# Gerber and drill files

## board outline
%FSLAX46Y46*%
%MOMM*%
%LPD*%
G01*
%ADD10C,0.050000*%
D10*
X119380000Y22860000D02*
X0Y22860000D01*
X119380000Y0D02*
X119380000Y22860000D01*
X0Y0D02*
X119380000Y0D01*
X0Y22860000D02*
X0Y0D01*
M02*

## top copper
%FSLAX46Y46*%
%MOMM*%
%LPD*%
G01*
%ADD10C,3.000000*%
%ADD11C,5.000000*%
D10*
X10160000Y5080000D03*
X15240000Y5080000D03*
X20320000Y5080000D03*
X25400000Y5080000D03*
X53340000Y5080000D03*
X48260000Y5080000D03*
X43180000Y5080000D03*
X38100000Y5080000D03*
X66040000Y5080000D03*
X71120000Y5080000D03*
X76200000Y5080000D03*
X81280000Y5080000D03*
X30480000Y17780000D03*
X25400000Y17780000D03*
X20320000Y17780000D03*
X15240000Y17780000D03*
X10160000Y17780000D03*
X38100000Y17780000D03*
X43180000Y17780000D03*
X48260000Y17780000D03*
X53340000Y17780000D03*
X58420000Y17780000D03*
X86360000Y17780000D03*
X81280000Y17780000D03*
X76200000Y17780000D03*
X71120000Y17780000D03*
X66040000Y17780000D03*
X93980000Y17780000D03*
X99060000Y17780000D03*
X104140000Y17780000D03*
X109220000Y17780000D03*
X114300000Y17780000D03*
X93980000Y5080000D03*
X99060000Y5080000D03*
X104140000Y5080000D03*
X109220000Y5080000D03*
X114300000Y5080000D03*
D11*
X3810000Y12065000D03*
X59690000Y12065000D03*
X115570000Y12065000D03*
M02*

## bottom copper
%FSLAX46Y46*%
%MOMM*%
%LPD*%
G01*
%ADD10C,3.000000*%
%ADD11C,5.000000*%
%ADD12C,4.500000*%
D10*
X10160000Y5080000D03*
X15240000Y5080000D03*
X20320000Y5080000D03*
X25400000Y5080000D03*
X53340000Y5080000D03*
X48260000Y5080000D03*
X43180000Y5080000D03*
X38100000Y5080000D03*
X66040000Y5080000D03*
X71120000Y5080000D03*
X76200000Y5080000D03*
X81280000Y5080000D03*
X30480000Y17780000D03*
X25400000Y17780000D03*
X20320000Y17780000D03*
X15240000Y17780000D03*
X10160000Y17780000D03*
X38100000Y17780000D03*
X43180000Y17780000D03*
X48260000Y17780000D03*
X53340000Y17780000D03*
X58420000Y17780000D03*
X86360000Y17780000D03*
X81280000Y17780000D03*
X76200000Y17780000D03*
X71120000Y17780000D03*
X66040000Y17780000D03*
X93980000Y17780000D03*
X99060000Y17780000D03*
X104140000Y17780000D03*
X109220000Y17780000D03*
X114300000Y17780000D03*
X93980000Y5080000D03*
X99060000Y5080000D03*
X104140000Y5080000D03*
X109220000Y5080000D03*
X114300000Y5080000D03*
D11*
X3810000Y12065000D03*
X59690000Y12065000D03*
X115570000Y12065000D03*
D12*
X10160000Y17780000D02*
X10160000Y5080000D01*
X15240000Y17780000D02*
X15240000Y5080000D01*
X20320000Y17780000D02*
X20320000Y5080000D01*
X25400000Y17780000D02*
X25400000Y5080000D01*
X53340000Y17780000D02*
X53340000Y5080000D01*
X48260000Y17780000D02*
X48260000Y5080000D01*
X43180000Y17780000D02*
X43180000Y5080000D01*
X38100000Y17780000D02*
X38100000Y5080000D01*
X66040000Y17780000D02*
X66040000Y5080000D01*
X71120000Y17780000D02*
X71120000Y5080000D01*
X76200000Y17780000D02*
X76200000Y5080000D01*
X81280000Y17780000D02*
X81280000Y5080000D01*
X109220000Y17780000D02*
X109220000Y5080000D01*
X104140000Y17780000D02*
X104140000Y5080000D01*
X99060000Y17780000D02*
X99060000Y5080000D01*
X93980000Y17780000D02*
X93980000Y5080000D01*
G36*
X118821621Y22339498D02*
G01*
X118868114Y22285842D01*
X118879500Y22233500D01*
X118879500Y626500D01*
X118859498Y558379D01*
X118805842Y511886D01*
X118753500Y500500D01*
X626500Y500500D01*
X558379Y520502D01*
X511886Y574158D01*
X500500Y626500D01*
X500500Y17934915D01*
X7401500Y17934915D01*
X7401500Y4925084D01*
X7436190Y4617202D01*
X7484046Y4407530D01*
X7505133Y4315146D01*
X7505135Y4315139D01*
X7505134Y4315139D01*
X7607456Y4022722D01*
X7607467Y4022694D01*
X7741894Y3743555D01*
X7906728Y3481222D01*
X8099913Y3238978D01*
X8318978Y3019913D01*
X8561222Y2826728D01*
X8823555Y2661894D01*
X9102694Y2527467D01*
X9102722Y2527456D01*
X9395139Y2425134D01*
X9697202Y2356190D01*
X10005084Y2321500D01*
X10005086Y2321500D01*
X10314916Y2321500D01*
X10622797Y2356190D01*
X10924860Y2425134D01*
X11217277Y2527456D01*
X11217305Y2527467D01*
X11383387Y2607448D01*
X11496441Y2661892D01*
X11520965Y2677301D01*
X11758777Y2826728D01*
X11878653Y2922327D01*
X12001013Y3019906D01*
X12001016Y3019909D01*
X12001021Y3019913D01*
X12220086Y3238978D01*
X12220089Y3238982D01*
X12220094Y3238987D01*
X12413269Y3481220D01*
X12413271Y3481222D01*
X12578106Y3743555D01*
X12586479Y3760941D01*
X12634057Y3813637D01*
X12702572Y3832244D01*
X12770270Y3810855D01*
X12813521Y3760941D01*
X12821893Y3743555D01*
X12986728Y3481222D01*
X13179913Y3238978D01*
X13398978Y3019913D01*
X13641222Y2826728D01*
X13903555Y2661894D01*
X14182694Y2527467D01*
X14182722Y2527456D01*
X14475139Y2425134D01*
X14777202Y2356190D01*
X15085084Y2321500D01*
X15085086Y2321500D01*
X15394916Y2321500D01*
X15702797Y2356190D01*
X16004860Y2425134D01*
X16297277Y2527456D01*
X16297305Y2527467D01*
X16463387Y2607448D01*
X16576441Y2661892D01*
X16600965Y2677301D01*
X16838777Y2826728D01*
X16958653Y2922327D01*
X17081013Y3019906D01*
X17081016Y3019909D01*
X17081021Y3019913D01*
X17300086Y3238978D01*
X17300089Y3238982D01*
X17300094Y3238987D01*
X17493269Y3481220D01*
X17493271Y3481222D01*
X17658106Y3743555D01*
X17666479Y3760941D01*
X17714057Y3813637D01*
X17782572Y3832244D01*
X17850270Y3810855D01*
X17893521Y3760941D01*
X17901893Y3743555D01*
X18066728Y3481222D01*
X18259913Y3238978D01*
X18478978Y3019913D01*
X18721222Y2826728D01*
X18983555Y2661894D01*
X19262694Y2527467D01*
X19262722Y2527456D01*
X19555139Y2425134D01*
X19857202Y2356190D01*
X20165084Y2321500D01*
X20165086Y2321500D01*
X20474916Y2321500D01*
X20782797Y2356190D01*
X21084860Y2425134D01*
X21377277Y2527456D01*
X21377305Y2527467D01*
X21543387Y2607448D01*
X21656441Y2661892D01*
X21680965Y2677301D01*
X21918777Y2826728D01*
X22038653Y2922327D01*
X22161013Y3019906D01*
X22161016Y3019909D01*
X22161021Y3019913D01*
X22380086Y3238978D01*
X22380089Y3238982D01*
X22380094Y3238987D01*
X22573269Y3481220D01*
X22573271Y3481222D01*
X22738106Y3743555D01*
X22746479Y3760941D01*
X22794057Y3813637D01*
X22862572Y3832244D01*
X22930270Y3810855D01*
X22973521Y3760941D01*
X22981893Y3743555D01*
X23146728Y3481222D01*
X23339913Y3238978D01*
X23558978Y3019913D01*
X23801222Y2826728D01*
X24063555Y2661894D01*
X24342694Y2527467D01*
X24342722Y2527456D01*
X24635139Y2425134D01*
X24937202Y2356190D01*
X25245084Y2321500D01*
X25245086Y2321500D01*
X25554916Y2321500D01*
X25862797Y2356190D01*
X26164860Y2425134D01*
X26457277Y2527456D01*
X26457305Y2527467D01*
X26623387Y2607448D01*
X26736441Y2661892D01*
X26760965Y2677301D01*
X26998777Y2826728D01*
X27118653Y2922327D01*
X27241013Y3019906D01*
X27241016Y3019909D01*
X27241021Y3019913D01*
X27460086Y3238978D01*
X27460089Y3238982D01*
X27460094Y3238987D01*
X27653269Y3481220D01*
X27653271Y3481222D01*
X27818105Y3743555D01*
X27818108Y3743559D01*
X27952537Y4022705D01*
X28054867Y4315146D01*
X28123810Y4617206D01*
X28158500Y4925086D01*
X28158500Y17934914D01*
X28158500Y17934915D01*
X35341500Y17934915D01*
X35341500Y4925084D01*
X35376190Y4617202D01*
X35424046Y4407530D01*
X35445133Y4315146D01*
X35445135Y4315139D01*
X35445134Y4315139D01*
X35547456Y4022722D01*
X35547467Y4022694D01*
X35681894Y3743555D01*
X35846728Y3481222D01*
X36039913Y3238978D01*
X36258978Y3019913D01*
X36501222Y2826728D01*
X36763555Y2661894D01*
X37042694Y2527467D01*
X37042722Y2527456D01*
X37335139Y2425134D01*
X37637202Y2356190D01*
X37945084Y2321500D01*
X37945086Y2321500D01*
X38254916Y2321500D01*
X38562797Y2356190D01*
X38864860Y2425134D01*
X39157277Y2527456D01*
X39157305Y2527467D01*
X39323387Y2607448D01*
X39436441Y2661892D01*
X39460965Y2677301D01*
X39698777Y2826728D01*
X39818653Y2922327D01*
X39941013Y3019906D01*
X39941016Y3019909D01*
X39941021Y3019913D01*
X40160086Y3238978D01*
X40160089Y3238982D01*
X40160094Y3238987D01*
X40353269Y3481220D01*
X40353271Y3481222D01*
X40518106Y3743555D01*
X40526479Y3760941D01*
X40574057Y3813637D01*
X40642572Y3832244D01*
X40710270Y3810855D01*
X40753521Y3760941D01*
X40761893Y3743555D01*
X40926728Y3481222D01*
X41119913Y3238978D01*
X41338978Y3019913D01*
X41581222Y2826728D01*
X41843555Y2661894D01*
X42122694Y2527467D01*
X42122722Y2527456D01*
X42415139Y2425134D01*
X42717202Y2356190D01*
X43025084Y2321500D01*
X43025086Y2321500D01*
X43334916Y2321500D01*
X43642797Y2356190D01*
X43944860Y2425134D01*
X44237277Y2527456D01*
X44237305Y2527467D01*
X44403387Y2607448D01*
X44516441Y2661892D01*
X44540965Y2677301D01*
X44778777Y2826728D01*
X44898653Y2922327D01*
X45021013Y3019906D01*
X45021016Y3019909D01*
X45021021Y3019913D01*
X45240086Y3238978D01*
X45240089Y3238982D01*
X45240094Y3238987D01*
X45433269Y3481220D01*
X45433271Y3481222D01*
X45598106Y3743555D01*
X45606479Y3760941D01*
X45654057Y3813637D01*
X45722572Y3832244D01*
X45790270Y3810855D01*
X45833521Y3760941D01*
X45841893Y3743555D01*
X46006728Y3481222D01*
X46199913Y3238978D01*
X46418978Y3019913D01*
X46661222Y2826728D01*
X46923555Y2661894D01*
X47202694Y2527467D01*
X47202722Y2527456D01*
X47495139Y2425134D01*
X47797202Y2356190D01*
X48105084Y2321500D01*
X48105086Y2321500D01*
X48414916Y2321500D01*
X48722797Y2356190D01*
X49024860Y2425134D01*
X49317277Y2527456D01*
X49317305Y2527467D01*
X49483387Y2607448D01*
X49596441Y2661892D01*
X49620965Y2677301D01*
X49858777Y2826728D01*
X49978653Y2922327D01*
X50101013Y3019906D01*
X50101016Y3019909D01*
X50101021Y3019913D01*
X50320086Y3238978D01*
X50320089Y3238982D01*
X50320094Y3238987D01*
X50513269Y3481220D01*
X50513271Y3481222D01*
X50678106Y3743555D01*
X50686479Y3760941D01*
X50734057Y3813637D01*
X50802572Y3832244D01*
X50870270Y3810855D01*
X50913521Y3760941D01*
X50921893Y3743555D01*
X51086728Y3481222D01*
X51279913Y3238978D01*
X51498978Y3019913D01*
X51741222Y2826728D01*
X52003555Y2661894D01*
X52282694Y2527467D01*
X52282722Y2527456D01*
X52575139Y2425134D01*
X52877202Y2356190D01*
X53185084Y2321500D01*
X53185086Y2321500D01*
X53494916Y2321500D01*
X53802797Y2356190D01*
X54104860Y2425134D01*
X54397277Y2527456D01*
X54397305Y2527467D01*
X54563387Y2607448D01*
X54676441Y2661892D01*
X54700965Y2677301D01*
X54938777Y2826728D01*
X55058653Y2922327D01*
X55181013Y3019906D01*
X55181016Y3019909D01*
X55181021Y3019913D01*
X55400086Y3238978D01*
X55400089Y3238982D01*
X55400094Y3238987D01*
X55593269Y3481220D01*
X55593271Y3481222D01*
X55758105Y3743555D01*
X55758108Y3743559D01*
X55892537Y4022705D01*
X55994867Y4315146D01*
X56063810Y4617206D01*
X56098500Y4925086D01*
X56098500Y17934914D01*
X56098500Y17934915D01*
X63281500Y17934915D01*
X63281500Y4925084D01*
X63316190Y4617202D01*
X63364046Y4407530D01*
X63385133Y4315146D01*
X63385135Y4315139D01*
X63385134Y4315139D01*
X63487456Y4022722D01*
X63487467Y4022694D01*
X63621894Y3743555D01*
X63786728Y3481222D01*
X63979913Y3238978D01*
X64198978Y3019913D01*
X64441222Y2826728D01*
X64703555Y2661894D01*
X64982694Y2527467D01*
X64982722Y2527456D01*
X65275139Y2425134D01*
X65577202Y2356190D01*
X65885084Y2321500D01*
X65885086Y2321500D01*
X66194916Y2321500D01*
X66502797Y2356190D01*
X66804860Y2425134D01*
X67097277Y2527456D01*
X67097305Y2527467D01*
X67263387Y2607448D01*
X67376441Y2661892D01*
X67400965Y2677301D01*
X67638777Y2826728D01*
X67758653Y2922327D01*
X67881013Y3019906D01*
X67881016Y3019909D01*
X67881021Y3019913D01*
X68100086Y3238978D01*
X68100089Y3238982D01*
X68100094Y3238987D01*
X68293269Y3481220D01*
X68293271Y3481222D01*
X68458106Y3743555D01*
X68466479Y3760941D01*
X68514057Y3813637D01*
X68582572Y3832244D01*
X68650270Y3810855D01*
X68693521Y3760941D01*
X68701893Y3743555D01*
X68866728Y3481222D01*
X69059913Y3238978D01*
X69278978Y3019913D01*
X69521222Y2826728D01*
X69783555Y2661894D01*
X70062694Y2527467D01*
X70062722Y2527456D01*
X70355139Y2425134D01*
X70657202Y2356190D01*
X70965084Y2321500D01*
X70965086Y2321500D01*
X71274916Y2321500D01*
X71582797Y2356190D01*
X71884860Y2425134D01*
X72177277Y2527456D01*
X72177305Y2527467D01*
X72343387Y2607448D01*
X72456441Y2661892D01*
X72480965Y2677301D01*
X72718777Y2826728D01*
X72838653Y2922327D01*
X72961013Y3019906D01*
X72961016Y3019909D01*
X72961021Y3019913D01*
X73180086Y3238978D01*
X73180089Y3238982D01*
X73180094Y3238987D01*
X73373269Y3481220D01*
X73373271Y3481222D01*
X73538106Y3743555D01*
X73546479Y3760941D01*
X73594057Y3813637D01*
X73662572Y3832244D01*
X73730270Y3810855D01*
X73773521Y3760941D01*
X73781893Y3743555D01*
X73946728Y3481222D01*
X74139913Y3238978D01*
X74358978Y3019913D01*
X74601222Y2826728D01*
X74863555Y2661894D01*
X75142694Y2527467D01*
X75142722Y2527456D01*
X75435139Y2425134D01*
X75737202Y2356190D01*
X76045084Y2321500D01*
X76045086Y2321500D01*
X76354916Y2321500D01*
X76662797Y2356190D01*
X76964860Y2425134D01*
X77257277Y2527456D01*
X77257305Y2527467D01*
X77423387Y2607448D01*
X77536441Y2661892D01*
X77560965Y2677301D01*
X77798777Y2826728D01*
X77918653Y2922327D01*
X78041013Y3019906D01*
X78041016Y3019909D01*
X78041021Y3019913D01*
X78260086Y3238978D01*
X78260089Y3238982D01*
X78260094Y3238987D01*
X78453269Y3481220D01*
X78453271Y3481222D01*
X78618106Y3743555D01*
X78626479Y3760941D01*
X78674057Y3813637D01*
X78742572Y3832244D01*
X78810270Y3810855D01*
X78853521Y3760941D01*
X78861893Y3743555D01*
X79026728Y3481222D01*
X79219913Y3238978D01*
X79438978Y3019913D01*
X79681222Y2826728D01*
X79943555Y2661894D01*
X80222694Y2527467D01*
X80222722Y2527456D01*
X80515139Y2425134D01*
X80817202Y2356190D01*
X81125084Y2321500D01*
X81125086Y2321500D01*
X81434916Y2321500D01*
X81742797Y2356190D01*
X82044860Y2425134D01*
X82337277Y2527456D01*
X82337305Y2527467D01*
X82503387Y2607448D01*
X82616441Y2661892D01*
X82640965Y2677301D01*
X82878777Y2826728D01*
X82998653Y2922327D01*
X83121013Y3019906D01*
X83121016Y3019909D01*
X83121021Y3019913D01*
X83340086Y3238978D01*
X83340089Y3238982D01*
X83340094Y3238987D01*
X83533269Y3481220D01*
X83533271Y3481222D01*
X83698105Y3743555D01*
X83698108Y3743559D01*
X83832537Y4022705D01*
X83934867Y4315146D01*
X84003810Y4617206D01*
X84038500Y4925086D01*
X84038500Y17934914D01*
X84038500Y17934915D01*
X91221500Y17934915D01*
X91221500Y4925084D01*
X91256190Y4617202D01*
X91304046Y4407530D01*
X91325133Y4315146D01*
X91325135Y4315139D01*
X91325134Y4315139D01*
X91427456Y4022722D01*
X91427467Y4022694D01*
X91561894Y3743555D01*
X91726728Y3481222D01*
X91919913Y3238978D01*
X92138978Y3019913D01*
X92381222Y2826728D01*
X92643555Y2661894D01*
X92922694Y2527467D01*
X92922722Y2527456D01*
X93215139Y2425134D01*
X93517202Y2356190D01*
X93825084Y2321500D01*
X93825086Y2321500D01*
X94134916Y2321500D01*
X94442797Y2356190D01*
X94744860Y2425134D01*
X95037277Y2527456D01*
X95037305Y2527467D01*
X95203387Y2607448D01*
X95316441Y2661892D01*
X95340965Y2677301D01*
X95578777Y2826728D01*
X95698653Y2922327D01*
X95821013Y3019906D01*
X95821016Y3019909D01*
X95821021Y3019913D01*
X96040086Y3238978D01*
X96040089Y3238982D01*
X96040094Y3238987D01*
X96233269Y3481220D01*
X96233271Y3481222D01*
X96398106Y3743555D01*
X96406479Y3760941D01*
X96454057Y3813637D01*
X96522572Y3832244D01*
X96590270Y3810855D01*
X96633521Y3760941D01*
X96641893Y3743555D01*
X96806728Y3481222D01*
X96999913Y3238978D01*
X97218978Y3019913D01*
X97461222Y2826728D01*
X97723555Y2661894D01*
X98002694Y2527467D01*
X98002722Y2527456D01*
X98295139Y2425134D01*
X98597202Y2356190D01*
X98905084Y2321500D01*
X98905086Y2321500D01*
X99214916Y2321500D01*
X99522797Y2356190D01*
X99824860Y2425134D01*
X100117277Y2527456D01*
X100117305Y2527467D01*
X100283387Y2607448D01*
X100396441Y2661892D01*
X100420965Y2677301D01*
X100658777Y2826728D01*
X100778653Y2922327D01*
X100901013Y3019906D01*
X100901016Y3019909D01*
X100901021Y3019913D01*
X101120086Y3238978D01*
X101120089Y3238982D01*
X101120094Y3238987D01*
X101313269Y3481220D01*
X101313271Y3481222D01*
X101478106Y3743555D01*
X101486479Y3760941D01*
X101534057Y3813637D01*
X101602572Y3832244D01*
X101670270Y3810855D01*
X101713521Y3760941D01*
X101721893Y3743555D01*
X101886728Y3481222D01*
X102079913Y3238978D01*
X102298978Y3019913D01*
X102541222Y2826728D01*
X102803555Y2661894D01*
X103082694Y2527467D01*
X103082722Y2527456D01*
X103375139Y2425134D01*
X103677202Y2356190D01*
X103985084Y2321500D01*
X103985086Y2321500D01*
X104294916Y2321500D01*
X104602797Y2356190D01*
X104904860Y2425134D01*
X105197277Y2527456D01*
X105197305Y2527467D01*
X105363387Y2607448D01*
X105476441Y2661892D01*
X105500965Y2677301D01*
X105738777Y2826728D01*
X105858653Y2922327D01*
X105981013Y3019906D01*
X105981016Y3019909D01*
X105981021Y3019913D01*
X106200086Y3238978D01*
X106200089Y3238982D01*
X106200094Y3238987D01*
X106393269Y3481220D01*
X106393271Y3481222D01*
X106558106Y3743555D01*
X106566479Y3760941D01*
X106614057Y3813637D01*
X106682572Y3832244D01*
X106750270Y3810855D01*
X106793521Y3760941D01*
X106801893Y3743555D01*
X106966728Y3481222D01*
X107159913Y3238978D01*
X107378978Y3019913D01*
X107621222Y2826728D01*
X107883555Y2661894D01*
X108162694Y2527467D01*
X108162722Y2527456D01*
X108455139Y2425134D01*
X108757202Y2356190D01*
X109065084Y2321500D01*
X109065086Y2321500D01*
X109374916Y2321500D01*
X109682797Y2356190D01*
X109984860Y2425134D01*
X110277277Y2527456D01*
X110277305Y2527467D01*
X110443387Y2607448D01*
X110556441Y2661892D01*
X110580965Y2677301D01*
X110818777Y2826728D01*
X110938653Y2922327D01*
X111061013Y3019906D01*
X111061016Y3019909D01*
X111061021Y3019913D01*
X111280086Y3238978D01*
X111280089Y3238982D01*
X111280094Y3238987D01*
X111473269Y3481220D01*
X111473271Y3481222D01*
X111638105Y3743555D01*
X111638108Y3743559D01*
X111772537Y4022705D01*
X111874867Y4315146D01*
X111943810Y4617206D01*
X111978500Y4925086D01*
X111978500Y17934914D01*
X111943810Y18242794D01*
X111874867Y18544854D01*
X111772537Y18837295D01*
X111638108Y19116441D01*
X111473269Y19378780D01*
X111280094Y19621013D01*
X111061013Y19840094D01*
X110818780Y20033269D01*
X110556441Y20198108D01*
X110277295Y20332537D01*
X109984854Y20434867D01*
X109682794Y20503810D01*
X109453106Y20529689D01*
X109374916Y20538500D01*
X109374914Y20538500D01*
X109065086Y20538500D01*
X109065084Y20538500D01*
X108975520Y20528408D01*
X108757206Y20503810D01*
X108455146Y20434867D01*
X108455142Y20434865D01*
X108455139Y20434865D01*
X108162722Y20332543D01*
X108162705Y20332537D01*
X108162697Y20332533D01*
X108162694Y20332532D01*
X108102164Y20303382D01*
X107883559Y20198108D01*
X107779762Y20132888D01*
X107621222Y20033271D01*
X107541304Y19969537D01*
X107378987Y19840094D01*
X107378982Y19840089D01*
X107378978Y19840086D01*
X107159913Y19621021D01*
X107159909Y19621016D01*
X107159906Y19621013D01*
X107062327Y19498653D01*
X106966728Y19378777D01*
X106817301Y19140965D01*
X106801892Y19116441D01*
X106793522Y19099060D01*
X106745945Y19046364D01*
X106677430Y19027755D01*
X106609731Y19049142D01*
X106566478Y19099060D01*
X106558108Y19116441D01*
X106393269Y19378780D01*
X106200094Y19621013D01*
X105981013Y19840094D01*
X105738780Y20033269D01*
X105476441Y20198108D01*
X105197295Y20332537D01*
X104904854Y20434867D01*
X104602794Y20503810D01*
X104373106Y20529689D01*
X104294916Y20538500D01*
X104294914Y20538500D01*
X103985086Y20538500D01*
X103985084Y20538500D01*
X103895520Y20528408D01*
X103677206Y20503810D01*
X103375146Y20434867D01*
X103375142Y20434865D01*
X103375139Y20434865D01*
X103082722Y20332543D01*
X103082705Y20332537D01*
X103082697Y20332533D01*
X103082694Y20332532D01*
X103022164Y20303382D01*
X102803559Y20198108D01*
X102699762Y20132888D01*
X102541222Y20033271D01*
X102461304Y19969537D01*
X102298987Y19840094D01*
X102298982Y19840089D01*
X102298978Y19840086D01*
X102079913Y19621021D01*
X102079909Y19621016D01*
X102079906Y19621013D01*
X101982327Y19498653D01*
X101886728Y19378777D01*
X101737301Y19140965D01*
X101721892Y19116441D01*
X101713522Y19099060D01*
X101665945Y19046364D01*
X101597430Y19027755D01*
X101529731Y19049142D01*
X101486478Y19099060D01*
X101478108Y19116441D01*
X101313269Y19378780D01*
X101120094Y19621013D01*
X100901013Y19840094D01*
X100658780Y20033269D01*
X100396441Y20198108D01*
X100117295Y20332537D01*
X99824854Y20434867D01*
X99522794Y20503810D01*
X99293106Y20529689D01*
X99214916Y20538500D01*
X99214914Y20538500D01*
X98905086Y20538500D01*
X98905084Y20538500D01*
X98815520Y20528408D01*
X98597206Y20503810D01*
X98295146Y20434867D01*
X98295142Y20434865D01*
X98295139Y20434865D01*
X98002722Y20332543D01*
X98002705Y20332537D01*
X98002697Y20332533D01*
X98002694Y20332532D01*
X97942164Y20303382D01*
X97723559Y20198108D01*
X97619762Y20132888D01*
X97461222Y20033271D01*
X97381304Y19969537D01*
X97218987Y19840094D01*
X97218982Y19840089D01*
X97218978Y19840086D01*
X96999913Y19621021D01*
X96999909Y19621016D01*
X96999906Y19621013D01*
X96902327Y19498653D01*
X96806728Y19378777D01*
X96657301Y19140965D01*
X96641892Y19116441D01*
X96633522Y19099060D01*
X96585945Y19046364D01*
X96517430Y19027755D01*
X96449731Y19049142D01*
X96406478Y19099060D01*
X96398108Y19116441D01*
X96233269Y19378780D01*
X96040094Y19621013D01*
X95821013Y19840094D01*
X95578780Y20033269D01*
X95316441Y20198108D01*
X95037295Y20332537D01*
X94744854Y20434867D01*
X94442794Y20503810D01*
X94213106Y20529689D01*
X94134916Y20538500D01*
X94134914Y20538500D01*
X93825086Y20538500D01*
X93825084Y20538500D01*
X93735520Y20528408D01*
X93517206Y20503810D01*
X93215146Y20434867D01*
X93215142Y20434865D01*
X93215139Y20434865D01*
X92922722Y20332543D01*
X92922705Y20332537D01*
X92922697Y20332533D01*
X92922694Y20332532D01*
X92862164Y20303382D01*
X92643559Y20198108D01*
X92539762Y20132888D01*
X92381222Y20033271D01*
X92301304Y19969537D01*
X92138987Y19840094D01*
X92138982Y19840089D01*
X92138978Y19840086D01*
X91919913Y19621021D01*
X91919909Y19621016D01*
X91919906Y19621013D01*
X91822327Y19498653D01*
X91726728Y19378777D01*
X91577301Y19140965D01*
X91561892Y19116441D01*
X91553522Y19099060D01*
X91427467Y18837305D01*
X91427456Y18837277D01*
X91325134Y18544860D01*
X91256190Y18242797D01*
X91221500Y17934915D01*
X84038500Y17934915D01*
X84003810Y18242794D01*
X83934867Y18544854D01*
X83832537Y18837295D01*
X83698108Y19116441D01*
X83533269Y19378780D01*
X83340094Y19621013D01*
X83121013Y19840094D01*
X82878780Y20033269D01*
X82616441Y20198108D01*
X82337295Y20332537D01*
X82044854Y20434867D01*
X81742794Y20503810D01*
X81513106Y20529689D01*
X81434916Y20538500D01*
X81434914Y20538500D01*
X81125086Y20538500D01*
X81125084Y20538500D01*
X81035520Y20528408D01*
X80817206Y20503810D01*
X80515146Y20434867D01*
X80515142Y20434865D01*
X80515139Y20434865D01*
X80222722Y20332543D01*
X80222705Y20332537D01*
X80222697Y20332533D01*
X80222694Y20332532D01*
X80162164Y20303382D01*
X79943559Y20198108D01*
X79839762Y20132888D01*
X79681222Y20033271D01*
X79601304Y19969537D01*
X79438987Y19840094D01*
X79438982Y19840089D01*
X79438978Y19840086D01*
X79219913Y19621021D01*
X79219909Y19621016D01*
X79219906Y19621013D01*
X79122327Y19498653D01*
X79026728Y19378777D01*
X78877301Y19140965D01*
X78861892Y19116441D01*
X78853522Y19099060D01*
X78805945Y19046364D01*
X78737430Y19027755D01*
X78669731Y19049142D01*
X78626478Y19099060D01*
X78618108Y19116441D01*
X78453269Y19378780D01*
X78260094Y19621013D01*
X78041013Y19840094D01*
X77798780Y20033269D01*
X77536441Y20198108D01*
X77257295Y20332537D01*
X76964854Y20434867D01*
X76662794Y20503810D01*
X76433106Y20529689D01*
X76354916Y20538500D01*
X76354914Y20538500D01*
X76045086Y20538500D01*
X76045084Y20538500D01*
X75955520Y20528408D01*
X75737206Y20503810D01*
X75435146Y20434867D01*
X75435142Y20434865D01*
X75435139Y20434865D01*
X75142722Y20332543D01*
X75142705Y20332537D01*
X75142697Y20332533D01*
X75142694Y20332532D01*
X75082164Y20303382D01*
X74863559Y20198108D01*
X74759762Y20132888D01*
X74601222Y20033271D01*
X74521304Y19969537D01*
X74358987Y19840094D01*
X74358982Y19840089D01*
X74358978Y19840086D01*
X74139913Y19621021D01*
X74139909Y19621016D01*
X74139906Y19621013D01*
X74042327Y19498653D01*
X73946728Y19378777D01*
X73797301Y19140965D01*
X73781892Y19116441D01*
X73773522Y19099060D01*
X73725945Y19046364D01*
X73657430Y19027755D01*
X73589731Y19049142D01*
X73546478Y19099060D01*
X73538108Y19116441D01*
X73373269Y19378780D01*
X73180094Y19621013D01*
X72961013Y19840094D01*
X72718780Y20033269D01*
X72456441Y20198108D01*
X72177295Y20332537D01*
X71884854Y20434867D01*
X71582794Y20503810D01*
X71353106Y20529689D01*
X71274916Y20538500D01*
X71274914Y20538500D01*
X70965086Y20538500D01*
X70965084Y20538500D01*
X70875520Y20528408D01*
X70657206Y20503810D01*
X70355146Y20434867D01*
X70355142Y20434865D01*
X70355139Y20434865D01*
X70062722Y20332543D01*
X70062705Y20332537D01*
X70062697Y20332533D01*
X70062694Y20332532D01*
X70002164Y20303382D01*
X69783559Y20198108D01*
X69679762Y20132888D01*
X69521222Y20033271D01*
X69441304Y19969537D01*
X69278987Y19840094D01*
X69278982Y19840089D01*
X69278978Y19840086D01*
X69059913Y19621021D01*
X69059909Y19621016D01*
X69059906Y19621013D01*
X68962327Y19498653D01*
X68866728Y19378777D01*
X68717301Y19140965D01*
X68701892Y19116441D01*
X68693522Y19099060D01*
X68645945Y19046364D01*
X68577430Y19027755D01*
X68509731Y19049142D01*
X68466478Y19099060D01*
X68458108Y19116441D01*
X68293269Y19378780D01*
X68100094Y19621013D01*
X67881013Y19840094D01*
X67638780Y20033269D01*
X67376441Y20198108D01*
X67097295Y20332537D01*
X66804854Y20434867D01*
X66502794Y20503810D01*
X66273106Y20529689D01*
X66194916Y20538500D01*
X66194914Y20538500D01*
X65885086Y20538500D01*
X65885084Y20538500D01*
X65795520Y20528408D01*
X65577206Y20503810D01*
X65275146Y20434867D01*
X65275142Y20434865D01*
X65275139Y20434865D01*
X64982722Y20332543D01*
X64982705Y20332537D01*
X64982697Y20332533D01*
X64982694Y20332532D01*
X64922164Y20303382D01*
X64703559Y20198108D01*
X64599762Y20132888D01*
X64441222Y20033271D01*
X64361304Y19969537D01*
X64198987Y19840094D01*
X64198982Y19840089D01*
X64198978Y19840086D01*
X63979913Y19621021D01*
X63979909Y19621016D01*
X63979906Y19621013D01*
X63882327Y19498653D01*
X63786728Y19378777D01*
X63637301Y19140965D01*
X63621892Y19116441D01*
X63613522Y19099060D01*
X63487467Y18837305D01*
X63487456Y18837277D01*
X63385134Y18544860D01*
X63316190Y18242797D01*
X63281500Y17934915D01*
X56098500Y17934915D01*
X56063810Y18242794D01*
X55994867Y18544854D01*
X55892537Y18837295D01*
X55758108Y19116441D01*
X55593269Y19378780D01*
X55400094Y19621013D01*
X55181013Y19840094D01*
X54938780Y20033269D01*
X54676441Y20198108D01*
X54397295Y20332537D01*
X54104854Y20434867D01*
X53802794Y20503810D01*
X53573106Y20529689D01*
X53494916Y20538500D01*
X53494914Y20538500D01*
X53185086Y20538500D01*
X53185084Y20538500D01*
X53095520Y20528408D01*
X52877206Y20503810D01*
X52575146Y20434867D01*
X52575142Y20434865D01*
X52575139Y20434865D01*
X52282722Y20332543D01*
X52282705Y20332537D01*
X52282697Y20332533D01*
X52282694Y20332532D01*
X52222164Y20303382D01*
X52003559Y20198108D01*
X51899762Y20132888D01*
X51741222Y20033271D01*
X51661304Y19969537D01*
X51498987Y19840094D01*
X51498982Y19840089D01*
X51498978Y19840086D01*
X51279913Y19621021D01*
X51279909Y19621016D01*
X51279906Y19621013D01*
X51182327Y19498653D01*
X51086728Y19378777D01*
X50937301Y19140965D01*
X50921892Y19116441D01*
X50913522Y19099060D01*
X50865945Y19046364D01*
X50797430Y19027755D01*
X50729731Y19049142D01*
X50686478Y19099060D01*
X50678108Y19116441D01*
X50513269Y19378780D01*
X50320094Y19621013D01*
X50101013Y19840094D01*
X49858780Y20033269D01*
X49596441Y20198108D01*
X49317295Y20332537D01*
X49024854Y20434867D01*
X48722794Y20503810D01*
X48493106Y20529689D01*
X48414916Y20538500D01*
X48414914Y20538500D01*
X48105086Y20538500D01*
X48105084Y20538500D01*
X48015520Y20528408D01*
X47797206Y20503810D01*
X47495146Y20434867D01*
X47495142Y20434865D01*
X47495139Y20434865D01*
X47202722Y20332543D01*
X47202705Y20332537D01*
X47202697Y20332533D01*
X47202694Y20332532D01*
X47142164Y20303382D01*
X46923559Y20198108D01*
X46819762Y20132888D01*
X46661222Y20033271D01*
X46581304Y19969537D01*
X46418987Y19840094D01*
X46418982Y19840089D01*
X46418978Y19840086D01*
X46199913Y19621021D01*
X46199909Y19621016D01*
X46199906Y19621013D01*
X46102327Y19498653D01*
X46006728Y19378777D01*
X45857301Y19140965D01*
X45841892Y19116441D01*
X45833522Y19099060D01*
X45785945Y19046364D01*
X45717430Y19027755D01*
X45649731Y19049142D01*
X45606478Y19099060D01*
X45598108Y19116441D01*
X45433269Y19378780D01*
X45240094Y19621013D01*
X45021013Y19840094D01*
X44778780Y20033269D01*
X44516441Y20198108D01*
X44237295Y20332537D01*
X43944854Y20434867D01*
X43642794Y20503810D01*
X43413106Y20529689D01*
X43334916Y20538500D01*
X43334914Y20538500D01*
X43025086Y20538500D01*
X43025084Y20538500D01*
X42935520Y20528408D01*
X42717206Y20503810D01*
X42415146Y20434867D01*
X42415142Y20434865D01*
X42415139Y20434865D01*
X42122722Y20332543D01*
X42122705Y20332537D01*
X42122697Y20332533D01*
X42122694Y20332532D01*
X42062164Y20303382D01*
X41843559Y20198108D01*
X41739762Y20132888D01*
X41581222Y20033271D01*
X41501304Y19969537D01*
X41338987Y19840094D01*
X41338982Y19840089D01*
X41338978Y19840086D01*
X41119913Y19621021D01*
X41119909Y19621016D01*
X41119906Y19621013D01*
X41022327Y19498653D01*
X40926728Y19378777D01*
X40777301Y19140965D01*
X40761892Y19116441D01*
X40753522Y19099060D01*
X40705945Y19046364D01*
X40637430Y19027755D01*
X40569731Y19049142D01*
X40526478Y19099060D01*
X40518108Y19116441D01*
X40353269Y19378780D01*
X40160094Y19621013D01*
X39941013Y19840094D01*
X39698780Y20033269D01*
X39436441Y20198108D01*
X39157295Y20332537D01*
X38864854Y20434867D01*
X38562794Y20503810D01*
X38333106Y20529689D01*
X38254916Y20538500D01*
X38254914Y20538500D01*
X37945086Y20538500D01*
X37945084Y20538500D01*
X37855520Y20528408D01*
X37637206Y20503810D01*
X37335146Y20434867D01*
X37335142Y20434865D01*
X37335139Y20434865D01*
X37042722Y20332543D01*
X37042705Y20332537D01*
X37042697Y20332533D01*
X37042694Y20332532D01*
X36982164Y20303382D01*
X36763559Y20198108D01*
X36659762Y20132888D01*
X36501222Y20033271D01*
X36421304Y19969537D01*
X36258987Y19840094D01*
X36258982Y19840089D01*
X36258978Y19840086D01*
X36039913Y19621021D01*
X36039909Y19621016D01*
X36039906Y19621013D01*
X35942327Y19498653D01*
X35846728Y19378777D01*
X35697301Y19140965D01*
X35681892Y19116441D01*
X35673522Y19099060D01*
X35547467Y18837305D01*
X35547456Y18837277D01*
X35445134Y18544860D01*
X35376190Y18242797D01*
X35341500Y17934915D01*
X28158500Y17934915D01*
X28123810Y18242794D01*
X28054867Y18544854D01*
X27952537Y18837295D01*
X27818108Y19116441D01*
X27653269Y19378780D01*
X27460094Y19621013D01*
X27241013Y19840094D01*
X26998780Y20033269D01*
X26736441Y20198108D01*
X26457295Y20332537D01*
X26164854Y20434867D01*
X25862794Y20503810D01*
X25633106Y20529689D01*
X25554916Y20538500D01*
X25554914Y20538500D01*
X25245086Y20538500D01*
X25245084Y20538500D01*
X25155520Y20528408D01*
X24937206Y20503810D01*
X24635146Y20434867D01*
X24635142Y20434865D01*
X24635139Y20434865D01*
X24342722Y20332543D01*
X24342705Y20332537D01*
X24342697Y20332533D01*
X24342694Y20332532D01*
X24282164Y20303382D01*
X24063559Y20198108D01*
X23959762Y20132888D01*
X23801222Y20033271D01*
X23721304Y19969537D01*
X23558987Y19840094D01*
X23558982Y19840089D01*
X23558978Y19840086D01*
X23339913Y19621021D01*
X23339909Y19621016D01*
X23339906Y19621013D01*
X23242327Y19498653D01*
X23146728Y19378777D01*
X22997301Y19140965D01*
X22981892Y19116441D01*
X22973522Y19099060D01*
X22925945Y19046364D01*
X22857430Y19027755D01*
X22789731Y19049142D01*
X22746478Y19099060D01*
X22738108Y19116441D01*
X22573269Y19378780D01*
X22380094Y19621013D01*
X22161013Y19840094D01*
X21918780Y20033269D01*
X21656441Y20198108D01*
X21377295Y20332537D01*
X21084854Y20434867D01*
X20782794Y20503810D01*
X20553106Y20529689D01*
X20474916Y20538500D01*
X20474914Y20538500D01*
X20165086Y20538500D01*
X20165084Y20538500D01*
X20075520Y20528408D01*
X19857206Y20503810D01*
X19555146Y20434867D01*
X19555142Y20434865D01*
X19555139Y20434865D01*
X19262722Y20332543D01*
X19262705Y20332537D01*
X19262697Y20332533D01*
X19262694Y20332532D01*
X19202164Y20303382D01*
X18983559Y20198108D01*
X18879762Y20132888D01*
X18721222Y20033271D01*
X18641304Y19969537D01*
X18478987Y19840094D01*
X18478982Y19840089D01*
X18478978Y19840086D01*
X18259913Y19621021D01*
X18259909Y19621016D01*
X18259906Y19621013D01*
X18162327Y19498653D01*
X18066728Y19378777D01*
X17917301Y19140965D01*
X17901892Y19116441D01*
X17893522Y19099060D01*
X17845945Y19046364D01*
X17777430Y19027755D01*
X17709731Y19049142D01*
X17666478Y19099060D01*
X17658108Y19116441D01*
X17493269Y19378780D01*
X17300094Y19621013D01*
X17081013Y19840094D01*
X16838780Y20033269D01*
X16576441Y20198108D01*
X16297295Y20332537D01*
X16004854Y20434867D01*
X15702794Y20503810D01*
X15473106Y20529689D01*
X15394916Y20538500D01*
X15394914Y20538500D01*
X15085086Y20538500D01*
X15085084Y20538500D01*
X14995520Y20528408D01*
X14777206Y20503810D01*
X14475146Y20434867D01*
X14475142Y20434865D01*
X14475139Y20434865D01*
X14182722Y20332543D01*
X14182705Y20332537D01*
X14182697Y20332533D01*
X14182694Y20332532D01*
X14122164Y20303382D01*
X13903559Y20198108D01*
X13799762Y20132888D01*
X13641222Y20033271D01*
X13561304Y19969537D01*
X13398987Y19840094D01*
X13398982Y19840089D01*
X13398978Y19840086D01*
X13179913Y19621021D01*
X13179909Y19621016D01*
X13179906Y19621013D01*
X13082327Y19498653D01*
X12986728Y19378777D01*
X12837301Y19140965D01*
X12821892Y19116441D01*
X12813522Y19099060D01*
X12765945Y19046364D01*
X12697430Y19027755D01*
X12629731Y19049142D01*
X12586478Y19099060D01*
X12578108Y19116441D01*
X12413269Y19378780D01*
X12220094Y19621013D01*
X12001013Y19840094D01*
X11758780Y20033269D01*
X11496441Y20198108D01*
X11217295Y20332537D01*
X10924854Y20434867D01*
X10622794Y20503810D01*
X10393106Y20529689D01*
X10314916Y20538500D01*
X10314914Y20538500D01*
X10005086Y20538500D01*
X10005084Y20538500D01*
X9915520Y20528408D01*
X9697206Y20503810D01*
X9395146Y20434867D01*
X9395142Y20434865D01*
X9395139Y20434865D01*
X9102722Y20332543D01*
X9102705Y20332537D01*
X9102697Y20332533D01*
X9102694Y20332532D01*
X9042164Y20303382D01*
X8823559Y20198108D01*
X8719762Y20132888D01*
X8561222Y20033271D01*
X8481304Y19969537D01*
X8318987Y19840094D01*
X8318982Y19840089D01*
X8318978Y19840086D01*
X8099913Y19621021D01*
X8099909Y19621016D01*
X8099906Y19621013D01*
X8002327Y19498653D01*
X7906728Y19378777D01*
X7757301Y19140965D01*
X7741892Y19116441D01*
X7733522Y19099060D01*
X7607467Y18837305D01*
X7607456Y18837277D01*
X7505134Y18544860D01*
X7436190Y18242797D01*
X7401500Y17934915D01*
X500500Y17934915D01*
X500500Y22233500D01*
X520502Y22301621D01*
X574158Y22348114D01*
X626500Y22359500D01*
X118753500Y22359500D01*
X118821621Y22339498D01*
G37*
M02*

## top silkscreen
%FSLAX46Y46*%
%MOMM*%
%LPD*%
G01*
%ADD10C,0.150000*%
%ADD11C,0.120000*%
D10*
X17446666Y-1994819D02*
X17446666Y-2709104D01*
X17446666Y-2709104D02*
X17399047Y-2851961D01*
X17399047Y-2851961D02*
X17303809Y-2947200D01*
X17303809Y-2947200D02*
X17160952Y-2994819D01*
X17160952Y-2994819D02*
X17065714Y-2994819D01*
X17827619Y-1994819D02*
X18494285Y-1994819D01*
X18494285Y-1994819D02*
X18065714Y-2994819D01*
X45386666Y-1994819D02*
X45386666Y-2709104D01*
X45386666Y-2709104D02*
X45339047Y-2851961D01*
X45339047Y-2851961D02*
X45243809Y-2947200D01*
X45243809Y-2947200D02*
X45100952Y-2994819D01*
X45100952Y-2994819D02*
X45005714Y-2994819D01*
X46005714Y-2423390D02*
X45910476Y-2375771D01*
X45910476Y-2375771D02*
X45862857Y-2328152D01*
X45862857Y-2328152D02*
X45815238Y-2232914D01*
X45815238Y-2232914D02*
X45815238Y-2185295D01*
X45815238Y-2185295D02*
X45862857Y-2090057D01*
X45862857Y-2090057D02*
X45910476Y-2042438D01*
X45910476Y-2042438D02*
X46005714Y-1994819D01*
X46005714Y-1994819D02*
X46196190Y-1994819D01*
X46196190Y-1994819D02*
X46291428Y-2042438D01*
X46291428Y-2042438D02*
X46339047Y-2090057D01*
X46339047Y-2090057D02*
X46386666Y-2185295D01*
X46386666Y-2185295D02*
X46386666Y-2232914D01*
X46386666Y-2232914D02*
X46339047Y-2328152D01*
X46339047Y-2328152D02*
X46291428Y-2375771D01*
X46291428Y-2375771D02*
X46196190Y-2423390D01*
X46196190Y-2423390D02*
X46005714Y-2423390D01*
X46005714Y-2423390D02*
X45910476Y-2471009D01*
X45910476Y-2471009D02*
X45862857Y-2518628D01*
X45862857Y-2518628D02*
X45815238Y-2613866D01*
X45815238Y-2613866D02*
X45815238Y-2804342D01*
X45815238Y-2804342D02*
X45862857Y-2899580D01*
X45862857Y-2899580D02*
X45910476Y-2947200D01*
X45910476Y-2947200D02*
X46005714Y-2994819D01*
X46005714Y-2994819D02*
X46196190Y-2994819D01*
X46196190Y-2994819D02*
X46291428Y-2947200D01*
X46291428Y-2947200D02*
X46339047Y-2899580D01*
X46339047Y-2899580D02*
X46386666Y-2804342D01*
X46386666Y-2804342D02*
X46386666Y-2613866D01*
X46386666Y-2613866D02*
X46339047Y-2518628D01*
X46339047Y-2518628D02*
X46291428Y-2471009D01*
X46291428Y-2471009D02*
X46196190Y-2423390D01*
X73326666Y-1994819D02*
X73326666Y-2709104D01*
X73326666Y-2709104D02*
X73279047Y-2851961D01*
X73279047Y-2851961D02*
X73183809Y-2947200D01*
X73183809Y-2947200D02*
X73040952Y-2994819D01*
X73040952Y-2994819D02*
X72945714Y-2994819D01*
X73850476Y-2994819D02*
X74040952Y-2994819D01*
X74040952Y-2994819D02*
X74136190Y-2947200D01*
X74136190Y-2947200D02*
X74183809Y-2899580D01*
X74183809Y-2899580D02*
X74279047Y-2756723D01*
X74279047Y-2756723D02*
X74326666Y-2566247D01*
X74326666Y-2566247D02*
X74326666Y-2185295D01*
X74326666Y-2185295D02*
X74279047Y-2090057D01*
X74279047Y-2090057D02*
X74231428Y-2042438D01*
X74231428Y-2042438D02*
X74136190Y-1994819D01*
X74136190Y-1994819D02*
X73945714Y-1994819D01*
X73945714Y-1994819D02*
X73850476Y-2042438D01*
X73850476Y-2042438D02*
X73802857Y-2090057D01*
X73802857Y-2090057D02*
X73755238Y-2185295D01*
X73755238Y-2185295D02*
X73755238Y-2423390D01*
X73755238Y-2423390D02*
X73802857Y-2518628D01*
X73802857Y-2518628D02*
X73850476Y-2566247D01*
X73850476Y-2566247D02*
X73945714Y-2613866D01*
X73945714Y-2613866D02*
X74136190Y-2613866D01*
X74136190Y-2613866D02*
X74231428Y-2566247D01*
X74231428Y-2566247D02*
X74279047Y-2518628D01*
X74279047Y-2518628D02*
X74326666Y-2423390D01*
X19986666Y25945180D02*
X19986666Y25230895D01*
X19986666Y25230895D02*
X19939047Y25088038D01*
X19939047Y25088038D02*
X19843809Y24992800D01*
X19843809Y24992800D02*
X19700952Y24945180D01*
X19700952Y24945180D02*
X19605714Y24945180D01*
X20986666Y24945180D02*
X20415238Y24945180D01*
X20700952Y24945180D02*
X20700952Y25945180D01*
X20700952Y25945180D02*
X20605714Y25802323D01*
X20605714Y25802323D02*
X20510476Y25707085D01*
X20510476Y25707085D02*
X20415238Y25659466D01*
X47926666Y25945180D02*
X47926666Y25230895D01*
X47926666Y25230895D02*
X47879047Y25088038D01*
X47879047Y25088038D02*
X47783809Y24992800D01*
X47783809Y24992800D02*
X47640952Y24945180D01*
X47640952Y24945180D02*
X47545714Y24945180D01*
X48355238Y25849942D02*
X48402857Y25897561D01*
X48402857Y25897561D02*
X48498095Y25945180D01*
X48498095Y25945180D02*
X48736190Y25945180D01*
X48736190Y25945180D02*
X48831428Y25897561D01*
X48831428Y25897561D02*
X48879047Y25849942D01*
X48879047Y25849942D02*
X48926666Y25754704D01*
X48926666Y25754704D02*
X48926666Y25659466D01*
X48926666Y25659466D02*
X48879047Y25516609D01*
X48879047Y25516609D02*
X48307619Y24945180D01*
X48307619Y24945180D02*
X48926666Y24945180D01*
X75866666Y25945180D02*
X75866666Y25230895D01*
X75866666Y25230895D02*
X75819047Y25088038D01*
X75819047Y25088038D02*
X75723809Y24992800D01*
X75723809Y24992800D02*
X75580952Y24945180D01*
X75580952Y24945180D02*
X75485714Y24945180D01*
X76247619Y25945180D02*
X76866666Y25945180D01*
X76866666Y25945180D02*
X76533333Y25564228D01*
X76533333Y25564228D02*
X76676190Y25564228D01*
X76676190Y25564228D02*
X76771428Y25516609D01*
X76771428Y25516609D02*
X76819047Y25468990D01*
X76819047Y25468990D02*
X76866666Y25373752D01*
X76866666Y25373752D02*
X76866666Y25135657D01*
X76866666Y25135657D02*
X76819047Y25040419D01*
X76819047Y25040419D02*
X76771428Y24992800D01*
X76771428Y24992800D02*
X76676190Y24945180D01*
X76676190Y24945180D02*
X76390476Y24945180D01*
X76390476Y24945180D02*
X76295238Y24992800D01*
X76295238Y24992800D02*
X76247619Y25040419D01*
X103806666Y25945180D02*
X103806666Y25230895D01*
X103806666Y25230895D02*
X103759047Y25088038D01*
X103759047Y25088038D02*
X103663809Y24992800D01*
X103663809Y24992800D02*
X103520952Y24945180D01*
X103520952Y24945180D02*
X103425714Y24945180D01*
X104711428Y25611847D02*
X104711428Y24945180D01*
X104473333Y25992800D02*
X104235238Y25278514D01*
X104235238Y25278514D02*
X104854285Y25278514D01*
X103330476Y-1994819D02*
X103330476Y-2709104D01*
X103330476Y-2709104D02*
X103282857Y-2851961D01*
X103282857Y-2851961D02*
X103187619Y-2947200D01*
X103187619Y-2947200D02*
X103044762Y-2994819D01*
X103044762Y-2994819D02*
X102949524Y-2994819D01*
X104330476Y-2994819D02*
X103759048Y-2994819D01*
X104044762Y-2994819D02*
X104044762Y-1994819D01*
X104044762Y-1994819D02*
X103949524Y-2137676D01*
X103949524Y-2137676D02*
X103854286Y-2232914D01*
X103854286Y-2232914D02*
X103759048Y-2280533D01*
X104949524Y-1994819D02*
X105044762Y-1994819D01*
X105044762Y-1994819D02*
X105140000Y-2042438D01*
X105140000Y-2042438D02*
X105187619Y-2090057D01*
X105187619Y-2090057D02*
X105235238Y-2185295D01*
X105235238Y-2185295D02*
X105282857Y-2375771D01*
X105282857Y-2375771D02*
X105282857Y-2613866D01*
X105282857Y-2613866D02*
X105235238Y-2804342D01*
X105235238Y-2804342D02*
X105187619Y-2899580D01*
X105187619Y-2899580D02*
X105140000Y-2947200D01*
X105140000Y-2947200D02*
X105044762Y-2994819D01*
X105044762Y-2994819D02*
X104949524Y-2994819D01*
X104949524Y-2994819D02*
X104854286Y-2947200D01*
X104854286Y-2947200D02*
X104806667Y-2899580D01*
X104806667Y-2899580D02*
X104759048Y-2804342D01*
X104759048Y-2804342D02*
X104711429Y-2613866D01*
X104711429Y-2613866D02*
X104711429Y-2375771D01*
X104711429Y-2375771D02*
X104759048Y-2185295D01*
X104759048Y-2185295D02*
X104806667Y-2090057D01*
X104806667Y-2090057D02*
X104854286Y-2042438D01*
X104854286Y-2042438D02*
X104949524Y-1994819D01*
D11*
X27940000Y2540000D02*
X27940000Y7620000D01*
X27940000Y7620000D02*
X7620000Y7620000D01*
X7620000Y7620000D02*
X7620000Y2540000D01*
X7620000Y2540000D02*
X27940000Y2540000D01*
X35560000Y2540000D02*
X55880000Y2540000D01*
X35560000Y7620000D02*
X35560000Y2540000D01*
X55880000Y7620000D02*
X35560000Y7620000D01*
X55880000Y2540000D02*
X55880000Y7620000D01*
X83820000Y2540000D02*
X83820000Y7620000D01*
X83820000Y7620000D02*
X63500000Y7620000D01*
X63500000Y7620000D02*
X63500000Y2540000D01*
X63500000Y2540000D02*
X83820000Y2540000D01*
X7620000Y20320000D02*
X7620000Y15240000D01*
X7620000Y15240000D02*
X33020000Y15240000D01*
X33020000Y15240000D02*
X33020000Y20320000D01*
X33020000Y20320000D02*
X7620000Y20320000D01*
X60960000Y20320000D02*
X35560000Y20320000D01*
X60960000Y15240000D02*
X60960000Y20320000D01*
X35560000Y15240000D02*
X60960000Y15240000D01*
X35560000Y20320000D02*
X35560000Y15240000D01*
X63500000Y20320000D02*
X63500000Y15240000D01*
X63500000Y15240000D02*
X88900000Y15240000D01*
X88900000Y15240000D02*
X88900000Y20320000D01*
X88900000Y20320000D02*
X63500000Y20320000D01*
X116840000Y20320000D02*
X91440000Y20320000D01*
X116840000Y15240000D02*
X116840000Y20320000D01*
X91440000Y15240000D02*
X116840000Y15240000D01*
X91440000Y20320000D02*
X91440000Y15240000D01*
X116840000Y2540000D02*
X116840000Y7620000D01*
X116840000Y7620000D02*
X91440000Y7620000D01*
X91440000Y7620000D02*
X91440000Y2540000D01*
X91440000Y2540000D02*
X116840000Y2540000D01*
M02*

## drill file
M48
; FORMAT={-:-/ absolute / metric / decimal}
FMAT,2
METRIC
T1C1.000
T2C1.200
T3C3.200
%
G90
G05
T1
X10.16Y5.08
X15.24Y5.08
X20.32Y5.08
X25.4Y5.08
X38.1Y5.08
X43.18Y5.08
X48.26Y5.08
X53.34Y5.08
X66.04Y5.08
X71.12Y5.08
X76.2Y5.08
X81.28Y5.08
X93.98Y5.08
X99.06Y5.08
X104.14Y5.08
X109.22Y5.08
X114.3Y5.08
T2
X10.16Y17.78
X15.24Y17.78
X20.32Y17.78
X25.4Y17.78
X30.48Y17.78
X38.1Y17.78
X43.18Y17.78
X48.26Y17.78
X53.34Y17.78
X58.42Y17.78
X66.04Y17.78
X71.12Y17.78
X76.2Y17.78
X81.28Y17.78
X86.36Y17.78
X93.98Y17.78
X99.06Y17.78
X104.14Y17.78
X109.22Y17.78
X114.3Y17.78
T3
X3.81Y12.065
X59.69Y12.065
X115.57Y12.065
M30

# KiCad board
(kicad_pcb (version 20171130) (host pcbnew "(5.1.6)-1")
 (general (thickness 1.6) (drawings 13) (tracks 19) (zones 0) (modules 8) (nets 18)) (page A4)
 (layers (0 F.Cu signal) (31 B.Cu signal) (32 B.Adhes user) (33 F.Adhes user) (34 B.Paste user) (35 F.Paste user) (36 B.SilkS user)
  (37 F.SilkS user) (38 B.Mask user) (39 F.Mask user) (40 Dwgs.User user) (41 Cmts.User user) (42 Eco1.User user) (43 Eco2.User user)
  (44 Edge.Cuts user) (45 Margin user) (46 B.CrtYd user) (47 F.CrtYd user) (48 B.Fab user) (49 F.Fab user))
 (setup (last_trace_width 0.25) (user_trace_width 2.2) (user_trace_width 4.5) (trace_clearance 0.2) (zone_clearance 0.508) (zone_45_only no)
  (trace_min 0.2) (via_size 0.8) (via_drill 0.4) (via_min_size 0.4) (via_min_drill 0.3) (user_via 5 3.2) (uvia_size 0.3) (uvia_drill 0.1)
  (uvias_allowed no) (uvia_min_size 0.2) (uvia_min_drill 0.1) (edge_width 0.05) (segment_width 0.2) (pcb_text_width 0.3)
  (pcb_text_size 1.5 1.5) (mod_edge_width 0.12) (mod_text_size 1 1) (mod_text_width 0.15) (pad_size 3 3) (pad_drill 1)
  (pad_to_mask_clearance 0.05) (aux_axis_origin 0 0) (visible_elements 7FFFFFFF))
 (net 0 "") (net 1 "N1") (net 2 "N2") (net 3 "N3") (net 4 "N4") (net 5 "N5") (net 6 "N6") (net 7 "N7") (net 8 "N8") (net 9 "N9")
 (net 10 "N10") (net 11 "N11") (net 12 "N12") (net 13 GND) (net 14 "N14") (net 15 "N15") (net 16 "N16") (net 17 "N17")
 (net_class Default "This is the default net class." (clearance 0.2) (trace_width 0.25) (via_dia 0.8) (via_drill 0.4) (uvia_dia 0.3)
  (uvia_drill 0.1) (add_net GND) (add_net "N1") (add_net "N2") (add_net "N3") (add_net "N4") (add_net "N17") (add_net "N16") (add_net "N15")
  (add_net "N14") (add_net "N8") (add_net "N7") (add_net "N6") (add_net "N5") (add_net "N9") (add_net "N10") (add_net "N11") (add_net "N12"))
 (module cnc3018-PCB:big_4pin (layer F.Cu) (at 17.78 -5.08 180)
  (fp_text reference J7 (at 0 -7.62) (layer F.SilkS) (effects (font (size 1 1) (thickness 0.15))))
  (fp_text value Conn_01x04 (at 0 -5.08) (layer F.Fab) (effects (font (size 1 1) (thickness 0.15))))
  (fp_line (start -10.16 -2.54) (end -10.16 2.54) (layer F.SilkS) (width 0.12))
  (fp_line (start -10.16 2.54) (end 10.16 2.54) (layer F.SilkS) (width 0.12))
  (fp_line (start 10.16 2.54) (end 10.16 -2.54) (layer F.SilkS) (width 0.12))
  (fp_line (start 10.16 -2.54) (end -10.16 -2.54) (layer F.SilkS) (width 0.12))
  (pad 4 thru_hole circle (at 7.62 0 180) (size 3 3) (drill 1) (layers *.Cu *.Mask) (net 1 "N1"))
  (pad 3 thru_hole circle (at 2.54 0 180) (size 3 3) (drill 1) (layers *.Cu *.Mask) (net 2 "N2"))
  (pad 2 thru_hole circle (at -2.54 0 180) (size 3 3) (drill 1) (layers *.Cu *.Mask) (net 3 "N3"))
  (pad 1 thru_hole circle (at -7.62 0 180) (size 3 3) (drill 1) (layers *.Cu *.Mask) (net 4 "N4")))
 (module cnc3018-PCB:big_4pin (layer F.Cu) (at 45.72 -5.08 180)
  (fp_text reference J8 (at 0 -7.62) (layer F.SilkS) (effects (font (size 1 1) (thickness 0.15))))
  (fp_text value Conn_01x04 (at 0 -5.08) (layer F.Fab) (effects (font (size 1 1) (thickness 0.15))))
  (fp_line (start 10.16 -2.54) (end -10.16 -2.54) (layer F.SilkS) (width 0.12))
  (fp_line (start 10.16 2.54) (end 10.16 -2.54) (layer F.SilkS) (width 0.12))
  (fp_line (start -10.16 2.54) (end 10.16 2.54) (layer F.SilkS) (width 0.12))
  (fp_line (start -10.16 -2.54) (end -10.16 2.54) (layer F.SilkS) (width 0.12))
  (pad 1 thru_hole circle (at -7.62 0 180) (size 3 3) (drill 1) (layers *.Cu *.Mask) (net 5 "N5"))
  (pad 2 thru_hole circle (at -2.54 0 180) (size 3 3) (drill 1) (layers *.Cu *.Mask) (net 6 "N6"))
  (pad 3 thru_hole circle (at 2.54 0 180) (size 3 3) (drill 1) (layers *.Cu *.Mask) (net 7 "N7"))
  (pad 4 thru_hole circle (at 7.62 0 180) (size 3 3) (drill 1) (layers *.Cu *.Mask) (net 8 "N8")))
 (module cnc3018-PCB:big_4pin (layer F.Cu) (at 73.66 -5.08 180)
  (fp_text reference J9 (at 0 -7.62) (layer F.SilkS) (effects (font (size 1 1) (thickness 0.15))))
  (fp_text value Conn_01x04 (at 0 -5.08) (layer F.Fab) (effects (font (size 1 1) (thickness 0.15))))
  (fp_line (start -10.16 -2.54) (end -10.16 2.54) (layer F.SilkS) (width 0.12))
  (fp_line (start -10.16 2.54) (end 10.16 2.54) (layer F.SilkS) (width 0.12))
  (fp_line (start 10.16 2.54) (end 10.16 -2.54) (layer F.SilkS) (width 0.12))
  (fp_line (start 10.16 -2.54) (end -10.16 -2.54) (layer F.SilkS) (width 0.12))
  (pad 4 thru_hole circle (at 7.62 0 180) (size 3 3) (drill 1) (layers *.Cu *.Mask) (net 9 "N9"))
  (pad 3 thru_hole circle (at 2.54 0 180) (size 3 3) (drill 1) (layers *.Cu *.Mask) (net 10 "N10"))
  (pad 2 thru_hole circle (at -2.54 0 180) (size 3 3) (drill 1) (layers *.Cu *.Mask) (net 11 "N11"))
  (pad 1 thru_hole circle (at -7.62 0 180) (size 3 3) (drill 1) (layers *.Cu *.Mask) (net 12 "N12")))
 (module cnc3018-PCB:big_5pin (layer F.Cu) (at 20.32 -17.78)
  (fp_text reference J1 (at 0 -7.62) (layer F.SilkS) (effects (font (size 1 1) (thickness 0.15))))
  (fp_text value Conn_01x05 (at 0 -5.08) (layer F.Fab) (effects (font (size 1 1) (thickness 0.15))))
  (fp_line (start -12.7 -2.54) (end -12.7 2.54) (layer F.SilkS) (width 0.12))
  (fp_line (start -12.7 2.54) (end 12.7 2.54) (layer F.SilkS) (width 0.12))
  (fp_line (start 12.7 2.54) (end 12.7 -2.54) (layer F.SilkS) (width 0.12))
  (fp_line (start 12.7 -2.54) (end -12.7 -2.54) (layer F.SilkS) (width 0.12))
  (pad 5 thru_hole circle (at 10.16 0) (size 3 3) (drill 1.2) (layers *.Cu *.Mask) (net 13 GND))
  (pad 4 thru_hole circle (at 5.08 0) (size 3 3) (drill 1.2) (layers *.Cu *.Mask) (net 4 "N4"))
  (pad 3 thru_hole circle (at 0 0) (size 3 3) (drill 1.2) (layers *.Cu *.Mask) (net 3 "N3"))
  (pad 2 thru_hole circle (at -5.08 0) (size 3 3) (drill 1.2) (layers *.Cu *.Mask) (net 2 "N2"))
  (pad 1 thru_hole circle (at -10.16 0) (size 3 3) (drill 1.2) (layers *.Cu *.Mask) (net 1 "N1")))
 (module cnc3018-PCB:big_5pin (layer F.Cu) (at 48.26 -17.78)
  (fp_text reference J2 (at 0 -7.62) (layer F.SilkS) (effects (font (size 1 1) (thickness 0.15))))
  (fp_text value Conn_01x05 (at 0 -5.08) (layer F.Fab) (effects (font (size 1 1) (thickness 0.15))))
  (fp_line (start 12.7 -2.54) (end -12.7 -2.54) (layer F.SilkS) (width 0.12))
  (fp_line (start 12.7 2.54) (end 12.7 -2.54) (layer F.SilkS) (width 0.12))
  (fp_line (start -12.7 2.54) (end 12.7 2.54) (layer F.SilkS) (width 0.12))
  (fp_line (start -12.7 -2.54) (end -12.7 2.54) (layer F.SilkS) (width 0.12))
  (pad 1 thru_hole circle (at -10.16 0) (size 3 3) (drill 1.2) (layers *.Cu *.Mask) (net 8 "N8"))
  (pad 2 thru_hole circle (at -5.08 0) (size 3 3) (drill 1.2) (layers *.Cu *.Mask) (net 7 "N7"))
  (pad 3 thru_hole circle (at 0 0) (size 3 3) (drill 1.2) (layers *.Cu *.Mask) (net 6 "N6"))
  (pad 4 thru_hole circle (at 5.08 0) (size 3 3) (drill 1.2) (layers *.Cu *.Mask) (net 5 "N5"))
  (pad 5 thru_hole circle (at 10.16 0) (size 3 3) (drill 1.2) (layers *.Cu *.Mask) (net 13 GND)))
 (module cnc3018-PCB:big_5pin (layer F.Cu) (at 76.2 -17.78)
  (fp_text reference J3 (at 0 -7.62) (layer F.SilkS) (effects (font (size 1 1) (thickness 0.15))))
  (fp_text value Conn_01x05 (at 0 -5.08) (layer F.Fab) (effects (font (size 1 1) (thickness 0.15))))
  (fp_line (start -12.7 -2.54) (end -12.7 2.54) (layer F.SilkS) (width 0.12))
  (fp_line (start -12.7 2.54) (end 12.7 2.54) (layer F.SilkS) (width 0.12))
  (fp_line (start 12.7 2.54) (end 12.7 -2.54) (layer F.SilkS) (width 0.12))
  (fp_line (start 12.7 -2.54) (end -12.7 -2.54) (layer F.SilkS) (width 0.12))
  (pad 5 thru_hole circle (at 10.16 0) (size 3 3) (drill 1.2) (layers *.Cu *.Mask) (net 13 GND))
  (pad 4 thru_hole circle (at 5.08 0) (size 3 3) (drill 1.2) (layers *.Cu *.Mask) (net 12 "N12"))
  (pad 3 thru_hole circle (at 0 0) (size 3 3) (drill 1.2) (layers *.Cu *.Mask) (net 11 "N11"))
  (pad 2 thru_hole circle (at -5.08 0) (size 3 3) (drill 1.2) (layers *.Cu *.Mask) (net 10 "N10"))
  (pad 1 thru_hole circle (at -10.16 0) (size 3 3) (drill 1.2) (layers *.Cu *.Mask) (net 9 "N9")))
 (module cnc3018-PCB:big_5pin (layer F.Cu) (at 104.14 -17.78)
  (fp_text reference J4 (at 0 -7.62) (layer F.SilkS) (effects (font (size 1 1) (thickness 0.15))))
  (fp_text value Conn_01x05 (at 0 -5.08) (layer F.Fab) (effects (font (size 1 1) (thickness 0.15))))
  (fp_line (start 12.7 -2.54) (end -12.7 -2.54) (layer F.SilkS) (width 0.12))
  (fp_line (start 12.7 2.54) (end 12.7 -2.54) (layer F.SilkS) (width 0.12))
  (fp_line (start -12.7 2.54) (end 12.7 2.54) (layer F.SilkS) (width 0.12))
  (fp_line (start -12.7 -2.54) (end -12.7 2.54) (layer F.SilkS) (width 0.12))
  (pad 1 thru_hole circle (at -10.16 0) (size 3 3) (drill 1.2) (layers *.Cu *.Mask) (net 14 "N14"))
  (pad 2 thru_hole circle (at -5.08 0) (size 3 3) (drill 1.2) (layers *.Cu *.Mask) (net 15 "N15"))
  (pad 3 thru_hole circle (at 0 0) (size 3 3) (drill 1.2) (layers *.Cu *.Mask) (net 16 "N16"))
  (pad 4 thru_hole circle (at 5.08 0) (size 3 3) (drill 1.2) (layers *.Cu *.Mask) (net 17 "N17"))
  (pad 5 thru_hole circle (at 10.16 0) (size 3 3) (drill 1.2) (layers *.Cu *.Mask) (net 13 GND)))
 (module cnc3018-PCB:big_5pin (layer F.Cu) (at 104.14 -5.08 180)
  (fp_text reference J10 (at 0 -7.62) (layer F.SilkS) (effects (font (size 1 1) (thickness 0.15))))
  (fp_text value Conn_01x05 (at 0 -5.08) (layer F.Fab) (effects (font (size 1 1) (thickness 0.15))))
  (fp_line (start -12.7 -2.54) (end -12.7 2.54) (layer F.SilkS) (width 0.12))
  (fp_line (start -12.7 2.54) (end 12.7 2.54) (layer F.SilkS) (width 0.12))
  (fp_line (start 12.7 2.54) (end 12.7 -2.54) (layer F.SilkS) (width 0.12))
  (fp_line (start 12.7 -2.54) (end -12.7 -2.54) (layer F.SilkS) (width 0.12))
  (pad 5 thru_hole circle (at 10.16 0 180) (size 3 3) (drill 1) (layers *.Cu *.Mask) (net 14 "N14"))
  (pad 4 thru_hole circle (at 5.08 0 180) (size 3 3) (drill 1) (layers *.Cu *.Mask) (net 15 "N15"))
  (pad 3 thru_hole circle (at 0 0 180) (size 3 3) (drill 1) (layers *.Cu *.Mask) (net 16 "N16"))
  (pad 2 thru_hole circle (at -5.08 0 180) (size 3 3) (drill 1) (layers *.Cu *.Mask) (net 17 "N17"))
  (pad 1 thru_hole circle (at -10.16 0 180) (size 3 3) (drill 1) (layers *.Cu *.Mask) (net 13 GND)))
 (gr_line (start 119.38 -22.86) (end 0 -22.86) (layer Edge.Cuts) (width 0.05))
 (gr_line (start 119.38 0) (end 119.38 -22.86) (layer Edge.Cuts) (width 0.05))
 (gr_line (start 0 0) (end 119.38 0) (layer Edge.Cuts) (width 0.05))
 (gr_line (start 0 -22.86) (end 0 0) (layer Edge.Cuts) (width 0.05))
 (segment (start 10.16 -17.78) (end 10.16 -5.08) (width 4.5) (layer B.Cu) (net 1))
 (segment (start 15.24 -17.78) (end 15.24 -5.08) (width 4.5) (layer B.Cu) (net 2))
 (segment (start 20.32 -17.78) (end 20.32 -5.08) (width 4.5) (layer B.Cu) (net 3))
 (segment (start 25.4 -17.78) (end 25.4 -5.08) (width 4.5) (layer B.Cu) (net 4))
 (segment (start 53.34 -17.78) (end 53.34 -5.08) (width 4.5) (layer B.Cu) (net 5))
 (segment (start 48.26 -17.78) (end 48.26 -5.08) (width 4.5) (layer B.Cu) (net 6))
 (segment (start 43.18 -17.78) (end 43.18 -5.08) (width 4.5) (layer B.Cu) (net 7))
 (segment (start 38.1 -17.78) (end 38.1 -5.08) (width 4.5) (layer B.Cu) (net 8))
 (segment (start 66.04 -17.78) (end 66.04 -5.08) (width 4.5) (layer B.Cu) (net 9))
 (segment (start 71.12 -17.78) (end 71.12 -5.08) (width 4.5) (layer B.Cu) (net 10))
 (segment (start 76.2 -17.78) (end 76.2 -5.08) (width 4.5) (layer B.Cu) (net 11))
 (segment (start 81.28 -17.78) (end 81.28 -5.08) (width 4.5) (layer B.Cu) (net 12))
 (segment (start 109.22 -17.78) (end 109.22 -5.08) (width 4.5) (layer B.Cu) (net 17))
 (segment (start 104.14 -17.78) (end 104.14 -5.08) (width 4.5) (layer B.Cu) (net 16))
 (segment (start 99.06 -17.78) (end 99.06 -5.08) (width 4.5) (layer B.Cu) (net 15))
 (segment (start 93.98 -17.78) (end 93.98 -5.08) (width 4.5) (layer B.Cu) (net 14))
 (via (at 3.81 -12.065) (size 5) (drill 3.2) (layers F.Cu B.Cu) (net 13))
 (via (at 59.69 -12.065) (size 5) (drill 3.2) (layers F.Cu B.Cu) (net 13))
 (via (at 115.57 -12.065) (size 5) (drill 3.2) (layers F.Cu B.Cu) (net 13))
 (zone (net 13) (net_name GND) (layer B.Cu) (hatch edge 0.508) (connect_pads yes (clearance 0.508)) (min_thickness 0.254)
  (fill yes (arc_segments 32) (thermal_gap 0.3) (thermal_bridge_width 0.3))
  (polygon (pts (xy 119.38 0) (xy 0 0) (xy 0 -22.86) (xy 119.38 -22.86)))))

